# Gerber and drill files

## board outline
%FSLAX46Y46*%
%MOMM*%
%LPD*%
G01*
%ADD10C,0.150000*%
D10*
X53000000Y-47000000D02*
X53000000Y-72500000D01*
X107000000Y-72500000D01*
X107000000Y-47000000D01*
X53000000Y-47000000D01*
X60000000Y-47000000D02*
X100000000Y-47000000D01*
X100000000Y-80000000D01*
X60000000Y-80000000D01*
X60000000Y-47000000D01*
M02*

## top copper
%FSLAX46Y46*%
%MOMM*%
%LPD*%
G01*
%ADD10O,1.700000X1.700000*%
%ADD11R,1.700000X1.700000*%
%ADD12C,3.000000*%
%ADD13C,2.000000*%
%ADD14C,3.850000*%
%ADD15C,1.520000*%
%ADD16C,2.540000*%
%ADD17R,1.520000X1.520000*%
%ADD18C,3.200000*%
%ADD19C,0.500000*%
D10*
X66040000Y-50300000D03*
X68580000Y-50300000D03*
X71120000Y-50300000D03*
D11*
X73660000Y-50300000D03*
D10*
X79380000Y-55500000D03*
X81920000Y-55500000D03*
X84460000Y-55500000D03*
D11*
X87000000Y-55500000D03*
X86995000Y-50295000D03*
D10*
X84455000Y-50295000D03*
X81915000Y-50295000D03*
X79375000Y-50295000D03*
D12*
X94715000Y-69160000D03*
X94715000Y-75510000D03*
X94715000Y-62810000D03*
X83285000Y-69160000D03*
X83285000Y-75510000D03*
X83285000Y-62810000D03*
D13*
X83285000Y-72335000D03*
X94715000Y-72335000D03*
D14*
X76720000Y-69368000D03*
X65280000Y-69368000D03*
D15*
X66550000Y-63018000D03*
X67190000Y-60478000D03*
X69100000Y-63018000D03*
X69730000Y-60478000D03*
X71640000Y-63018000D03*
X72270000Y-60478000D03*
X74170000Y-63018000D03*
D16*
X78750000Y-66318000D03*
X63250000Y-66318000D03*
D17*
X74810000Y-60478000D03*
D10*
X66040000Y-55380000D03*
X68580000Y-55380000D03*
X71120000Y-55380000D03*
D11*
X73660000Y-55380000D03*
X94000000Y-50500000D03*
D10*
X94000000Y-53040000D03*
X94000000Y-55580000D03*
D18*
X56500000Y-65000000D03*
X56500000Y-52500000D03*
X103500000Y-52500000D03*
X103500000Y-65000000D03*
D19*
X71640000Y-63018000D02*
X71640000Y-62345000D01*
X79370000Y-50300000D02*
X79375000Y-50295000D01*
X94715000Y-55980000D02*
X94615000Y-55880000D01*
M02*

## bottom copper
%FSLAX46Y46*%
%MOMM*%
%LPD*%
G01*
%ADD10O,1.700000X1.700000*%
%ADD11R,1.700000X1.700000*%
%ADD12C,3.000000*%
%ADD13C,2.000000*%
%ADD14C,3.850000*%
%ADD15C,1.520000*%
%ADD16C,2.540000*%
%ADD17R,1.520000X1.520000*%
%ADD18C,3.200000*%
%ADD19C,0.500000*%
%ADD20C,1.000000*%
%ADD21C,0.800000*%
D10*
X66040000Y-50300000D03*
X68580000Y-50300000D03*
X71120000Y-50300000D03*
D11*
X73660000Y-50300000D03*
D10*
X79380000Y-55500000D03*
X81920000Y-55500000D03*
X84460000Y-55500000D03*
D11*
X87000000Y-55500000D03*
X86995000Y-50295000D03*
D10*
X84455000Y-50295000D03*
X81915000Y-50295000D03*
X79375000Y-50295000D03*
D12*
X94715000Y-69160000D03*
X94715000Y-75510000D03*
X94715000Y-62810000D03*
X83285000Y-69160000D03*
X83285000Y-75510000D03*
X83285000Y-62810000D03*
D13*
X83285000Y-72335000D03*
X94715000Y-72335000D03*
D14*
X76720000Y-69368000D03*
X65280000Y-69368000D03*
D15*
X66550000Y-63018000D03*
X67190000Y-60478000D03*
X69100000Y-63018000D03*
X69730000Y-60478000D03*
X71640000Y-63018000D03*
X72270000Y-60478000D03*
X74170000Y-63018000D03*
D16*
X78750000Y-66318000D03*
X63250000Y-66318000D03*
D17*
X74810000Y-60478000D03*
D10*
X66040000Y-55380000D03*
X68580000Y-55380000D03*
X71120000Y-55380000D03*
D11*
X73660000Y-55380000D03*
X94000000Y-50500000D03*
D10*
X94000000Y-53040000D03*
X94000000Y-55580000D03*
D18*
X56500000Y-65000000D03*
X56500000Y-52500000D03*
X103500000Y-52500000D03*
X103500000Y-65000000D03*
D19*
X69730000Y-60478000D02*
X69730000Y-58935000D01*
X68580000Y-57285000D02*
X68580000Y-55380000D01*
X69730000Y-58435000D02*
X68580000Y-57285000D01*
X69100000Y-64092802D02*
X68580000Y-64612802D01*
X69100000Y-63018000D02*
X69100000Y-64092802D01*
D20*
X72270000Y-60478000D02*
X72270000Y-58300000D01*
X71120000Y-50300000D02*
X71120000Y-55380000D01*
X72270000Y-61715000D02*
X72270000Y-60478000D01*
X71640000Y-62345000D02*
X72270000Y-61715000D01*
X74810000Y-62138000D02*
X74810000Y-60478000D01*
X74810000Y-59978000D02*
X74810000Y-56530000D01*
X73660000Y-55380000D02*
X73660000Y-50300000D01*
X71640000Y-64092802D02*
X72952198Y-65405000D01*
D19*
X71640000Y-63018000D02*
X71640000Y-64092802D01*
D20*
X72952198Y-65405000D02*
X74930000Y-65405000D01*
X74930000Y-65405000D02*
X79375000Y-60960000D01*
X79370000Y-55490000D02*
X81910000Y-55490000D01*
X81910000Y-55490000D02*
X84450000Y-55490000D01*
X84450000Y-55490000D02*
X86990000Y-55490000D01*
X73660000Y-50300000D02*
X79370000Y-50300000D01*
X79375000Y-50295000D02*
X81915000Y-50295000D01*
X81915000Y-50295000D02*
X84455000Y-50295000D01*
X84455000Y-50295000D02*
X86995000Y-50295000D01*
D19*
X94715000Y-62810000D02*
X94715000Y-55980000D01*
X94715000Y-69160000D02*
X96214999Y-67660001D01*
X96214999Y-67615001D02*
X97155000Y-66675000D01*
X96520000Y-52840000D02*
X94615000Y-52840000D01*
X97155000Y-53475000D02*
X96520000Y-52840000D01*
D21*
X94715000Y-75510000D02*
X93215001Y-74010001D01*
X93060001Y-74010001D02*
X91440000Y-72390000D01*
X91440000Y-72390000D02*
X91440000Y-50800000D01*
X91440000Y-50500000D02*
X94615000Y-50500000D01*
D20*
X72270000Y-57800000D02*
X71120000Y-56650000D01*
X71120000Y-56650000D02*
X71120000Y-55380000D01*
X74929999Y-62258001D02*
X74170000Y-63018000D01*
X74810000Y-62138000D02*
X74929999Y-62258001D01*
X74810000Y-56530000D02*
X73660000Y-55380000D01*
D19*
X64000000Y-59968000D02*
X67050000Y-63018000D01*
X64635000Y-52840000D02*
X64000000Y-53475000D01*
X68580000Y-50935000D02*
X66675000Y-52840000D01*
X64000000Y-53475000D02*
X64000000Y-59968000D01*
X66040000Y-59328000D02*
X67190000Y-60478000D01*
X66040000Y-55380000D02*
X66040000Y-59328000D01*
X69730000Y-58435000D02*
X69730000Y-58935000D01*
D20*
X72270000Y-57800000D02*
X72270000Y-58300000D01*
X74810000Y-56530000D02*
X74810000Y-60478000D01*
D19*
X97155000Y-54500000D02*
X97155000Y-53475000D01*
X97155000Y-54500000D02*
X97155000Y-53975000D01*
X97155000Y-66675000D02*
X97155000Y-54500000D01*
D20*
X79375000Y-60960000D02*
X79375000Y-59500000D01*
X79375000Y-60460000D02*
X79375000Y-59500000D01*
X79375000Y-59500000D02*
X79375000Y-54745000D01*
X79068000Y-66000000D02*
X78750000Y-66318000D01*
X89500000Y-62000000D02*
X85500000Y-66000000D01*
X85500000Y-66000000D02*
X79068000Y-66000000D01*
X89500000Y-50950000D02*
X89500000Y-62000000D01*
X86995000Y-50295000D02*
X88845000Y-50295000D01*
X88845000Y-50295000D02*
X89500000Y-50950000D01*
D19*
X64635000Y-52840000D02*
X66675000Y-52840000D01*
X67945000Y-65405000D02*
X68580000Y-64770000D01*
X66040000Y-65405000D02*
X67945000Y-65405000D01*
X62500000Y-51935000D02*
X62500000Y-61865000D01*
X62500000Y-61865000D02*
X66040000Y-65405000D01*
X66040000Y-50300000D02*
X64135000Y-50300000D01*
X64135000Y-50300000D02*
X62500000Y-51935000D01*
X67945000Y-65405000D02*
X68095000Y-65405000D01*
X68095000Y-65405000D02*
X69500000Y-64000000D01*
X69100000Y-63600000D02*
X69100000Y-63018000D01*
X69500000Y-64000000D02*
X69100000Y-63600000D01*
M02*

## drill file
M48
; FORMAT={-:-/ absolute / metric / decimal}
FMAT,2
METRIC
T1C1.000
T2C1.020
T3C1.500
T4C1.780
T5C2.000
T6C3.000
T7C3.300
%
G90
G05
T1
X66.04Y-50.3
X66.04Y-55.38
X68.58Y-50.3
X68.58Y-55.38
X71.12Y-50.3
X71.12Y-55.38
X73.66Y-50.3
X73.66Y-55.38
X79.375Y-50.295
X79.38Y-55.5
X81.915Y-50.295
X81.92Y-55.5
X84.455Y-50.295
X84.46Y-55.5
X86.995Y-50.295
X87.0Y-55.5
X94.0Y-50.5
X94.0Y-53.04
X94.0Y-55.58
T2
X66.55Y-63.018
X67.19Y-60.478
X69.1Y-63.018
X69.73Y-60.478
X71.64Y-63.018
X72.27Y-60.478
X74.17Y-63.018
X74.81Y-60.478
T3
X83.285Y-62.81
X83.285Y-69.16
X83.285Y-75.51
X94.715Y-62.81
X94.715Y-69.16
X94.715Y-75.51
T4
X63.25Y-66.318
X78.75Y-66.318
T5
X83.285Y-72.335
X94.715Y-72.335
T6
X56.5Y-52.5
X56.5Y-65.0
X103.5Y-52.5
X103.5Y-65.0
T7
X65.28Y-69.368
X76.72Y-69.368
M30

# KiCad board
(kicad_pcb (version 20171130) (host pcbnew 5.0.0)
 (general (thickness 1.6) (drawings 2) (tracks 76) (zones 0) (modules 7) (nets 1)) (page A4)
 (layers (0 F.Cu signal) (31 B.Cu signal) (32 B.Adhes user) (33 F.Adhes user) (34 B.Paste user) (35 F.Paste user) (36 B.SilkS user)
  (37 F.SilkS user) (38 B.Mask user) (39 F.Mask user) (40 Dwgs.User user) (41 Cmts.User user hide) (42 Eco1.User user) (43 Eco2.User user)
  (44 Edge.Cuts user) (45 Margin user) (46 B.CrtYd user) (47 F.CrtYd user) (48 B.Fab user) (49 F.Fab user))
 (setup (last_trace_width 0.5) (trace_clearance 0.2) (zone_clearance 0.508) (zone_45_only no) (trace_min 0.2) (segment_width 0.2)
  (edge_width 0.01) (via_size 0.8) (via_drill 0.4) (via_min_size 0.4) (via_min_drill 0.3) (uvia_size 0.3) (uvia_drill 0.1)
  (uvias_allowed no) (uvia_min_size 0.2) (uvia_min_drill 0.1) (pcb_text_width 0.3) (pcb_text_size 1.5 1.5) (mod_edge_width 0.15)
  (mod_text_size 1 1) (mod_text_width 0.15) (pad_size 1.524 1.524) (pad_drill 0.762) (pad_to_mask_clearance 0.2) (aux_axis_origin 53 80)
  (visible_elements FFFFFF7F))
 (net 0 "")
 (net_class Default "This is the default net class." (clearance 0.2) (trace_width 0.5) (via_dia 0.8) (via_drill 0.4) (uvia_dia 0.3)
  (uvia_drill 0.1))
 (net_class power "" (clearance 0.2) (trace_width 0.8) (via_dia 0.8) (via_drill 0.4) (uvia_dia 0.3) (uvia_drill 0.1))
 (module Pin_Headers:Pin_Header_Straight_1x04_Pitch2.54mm (layer F.Cu) (at 73.66 50.3 270)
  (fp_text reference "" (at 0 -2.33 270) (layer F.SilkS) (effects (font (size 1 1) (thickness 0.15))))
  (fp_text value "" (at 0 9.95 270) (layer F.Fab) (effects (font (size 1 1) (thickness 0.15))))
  (pad 4 thru_hole oval (at 0 7.62 270) (size 1.7 1.7) (drill 1) (layers *.Cu *.Mask))
  (pad 3 thru_hole oval (at 0 5.08 270) (size 1.7 1.7) (drill 1) (layers *.Cu *.Mask))
  (pad 2 thru_hole oval (at 0 2.54 270) (size 1.7 1.7) (drill 1) (layers *.Cu *.Mask))
  (pad 1 thru_hole rect (at 0 0 270) (size 1.7 1.7) (drill 1) (layers *.Cu *.Mask)))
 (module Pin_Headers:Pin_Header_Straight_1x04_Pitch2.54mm (layer F.Cu) (at 87 55.5 270)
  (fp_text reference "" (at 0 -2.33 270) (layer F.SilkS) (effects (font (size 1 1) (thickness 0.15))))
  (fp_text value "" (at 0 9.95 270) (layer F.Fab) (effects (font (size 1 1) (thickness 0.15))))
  (pad 4 thru_hole oval (at 0 7.62 270) (size 1.7 1.7) (drill 1) (layers *.Cu *.Mask))
  (pad 3 thru_hole oval (at 0 5.08 270) (size 1.7 1.7) (drill 1) (layers *.Cu *.Mask))
  (pad 2 thru_hole oval (at 0 2.54 270) (size 1.7 1.7) (drill 1) (layers *.Cu *.Mask))
  (pad 1 thru_hole rect (at 0 0 270) (size 1.7 1.7) (drill 1) (layers *.Cu *.Mask)))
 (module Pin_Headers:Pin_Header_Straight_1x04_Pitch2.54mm (layer F.Cu) (at 86.995 50.295 270)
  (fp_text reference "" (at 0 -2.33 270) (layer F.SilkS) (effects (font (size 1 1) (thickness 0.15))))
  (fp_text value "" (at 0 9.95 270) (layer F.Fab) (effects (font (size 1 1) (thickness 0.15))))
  (pad 1 thru_hole rect (at 0 0 270) (size 1.7 1.7) (drill 1) (layers *.Cu *.Mask))
  (pad 2 thru_hole oval (at 0 2.54 270) (size 1.7 1.7) (drill 1) (layers *.Cu *.Mask))
  (pad 3 thru_hole oval (at 0 5.08 270) (size 1.7 1.7) (drill 1) (layers *.Cu *.Mask))
  (pad 4 thru_hole oval (at 0 7.62 270) (size 1.7 1.7) (drill 1) (layers *.Cu *.Mask)))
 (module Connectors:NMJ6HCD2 (layer F.Cu) (at 89 59)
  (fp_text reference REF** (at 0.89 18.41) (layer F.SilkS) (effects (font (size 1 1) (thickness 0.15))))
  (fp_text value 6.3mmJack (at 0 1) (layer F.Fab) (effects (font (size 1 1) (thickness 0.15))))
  (pad 6 thru_hole circle (at 5.715 10.16) (size 3 3) (drill 1.5) (layers *.Cu *.Mask))
  (pad 5 thru_hole circle (at 5.715 16.51) (size 3 3) (drill 1.5) (layers *.Cu *.Mask))
  (pad 4 thru_hole circle (at 5.715 3.81) (size 3 3) (drill 1.5) (layers *.Cu *.Mask))
  (pad 3 thru_hole circle (at -5.715 10.16) (size 3 3) (drill 1.5) (layers *.Cu *.Mask))
  (pad 2 thru_hole circle (at -5.715 16.51) (size 3 3) (drill 1.5) (layers *.Cu *.Mask))
  (pad 1 thru_hole circle (at -5.715 3.81) (size 3 3) (drill 1.5) (layers *.Cu *.Mask))
  (pad "" thru_hole circle (at -5.715 13.335) (size 2 2) (drill 2) (layers *.Cu *.Mask))
  (pad "" thru_hole circle (at 5.715 13.335) (size 2 2) (drill 2) (layers *.Cu *.Mask)))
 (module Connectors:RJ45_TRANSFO (layer F.Cu) (at 71 59)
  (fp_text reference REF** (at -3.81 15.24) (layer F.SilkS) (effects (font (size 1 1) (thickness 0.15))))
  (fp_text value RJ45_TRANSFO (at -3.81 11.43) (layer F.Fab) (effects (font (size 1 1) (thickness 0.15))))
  (pad Hole thru_hole circle (at 5.72 10.368) (size 3.85 3.85) (drill 3.3) (layers *.Cu *.SilkS *.Mask))
  (pad Hole thru_hole circle (at -5.72 10.368) (size 3.85 3.85) (drill 3.3) (layers *.Cu *.SilkS *.Mask))
  (pad 8 thru_hole circle (at -4.45 4.018) (size 1.52 1.52) (drill 1.02) (layers *.Cu *.Mask))
  (pad 7 thru_hole circle (at -3.81 1.478) (size 1.52 1.52) (drill 1.02) (layers *.Cu *.Mask))
  (pad 6 thru_hole circle (at -1.9 4.018) (size 1.52 1.52) (drill 1.02) (layers *.Cu *.Mask))
  (pad 5 thru_hole circle (at -1.27 1.478) (size 1.52 1.52) (drill 1.02) (layers *.Cu *.Mask))
  (pad 4 thru_hole circle (at 0.64 4.018) (size 1.52 1.52) (drill 1.02) (layers *.Cu *.Mask))
  (pad 3 thru_hole circle (at 1.27 1.478) (size 1.52 1.52) (drill 1.02) (layers *.Cu *.Mask))
  (pad 2 thru_hole circle (at 3.17 4.018) (size 1.52 1.52) (drill 1.02) (layers *.Cu *.Mask))
  (pad 13 thru_hole circle (at 7.75 7.318) (size 2.54 2.54) (drill 1.78) (layers *.Cu *.SilkS *.Mask))
  (pad 13 thru_hole circle (at -7.75 7.318) (size 2.54 2.54) (drill 1.78) (layers *.Cu *.SilkS *.Mask))
  (pad 1 thru_hole rect (at 3.81 1.478) (size 1.52 1.52) (drill 1.02) (layers *.Cu *.Mask)))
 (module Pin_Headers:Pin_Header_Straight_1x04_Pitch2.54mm (layer F.Cu) (at 73.66 55.38 270)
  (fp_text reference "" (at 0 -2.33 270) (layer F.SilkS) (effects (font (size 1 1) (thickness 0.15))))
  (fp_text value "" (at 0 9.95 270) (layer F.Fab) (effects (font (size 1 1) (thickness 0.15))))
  (pad 4 thru_hole oval (at 0 7.62 270) (size 1.7 1.7) (drill 1) (layers *.Cu *.Mask))
  (pad 3 thru_hole oval (at 0 5.08 270) (size 1.7 1.7) (drill 1) (layers *.Cu *.Mask))
  (pad 2 thru_hole oval (at 0 2.54 270) (size 1.7 1.7) (drill 1) (layers *.Cu *.Mask))
  (pad 1 thru_hole rect (at 0 0 270) (size 1.7 1.7) (drill 1) (layers *.Cu *.Mask)))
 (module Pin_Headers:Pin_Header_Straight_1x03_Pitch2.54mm (layer F.Cu) (at 94 50.5)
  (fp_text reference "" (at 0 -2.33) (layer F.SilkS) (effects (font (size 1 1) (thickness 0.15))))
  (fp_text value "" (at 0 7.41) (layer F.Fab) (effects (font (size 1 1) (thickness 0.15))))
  (pad 1 thru_hole rect (at 0 0) (size 1.7 1.7) (drill 1) (layers *.Cu *.Mask))
  (pad 2 thru_hole oval (at 0 2.54) (size 1.7 1.7) (drill 1) (layers *.Cu *.Mask))
  (pad 3 thru_hole oval (at 0 5.08) (size 1.7 1.7) (drill 1) (layers *.Cu *.Mask)))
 (gr_poly (pts (xy 53 47) (xy 53 72.5) (xy 107 72.5) (xy 107 47)) (layer Edge.Cuts) (width 0.15))
 (gr_poly (pts (xy 60 47) (xy 100 47) (xy 100 80) (xy 60 80)) (layer Edge.Cuts) (width 0.15))
 (segment (start 69.73 60.478) (end 69.73 58.935) (width 0.5) (layer B.Cu) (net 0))
 (segment (start 68.58 57.285) (end 68.58 55.38) (width 0.5) (layer B.Cu) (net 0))
 (segment (start 69.73 58.435) (end 68.58 57.285) (width 0.5) (layer B.Cu) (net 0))
 (segment (start 69.1 64.092802) (end 68.58 64.612802) (width 0.5) (layer B.Cu) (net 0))
 (segment (start 69.1 63.018) (end 69.1 64.092802) (width 0.5) (layer B.Cu) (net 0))
 (segment (start 72.27 60.478) (end 72.27 58.3) (width 1) (layer B.Cu) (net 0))
 (segment (start 71.12 50.3) (end 71.12 55.38) (width 1) (layer B.Cu) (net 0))
 (segment (start 71.64 63.018) (end 71.64 62.345) (width 0.5) (layer F.Cu) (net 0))
 (segment (start 72.27 61.715) (end 72.27 60.478) (width 1) (layer B.Cu) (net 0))
 (segment (start 71.64 62.345) (end 72.27 61.715) (width 1) (layer B.Cu) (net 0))
 (segment (start 74.81 62.138) (end 74.81 60.478) (width 1) (layer B.Cu) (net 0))
 (segment (start 74.81 59.978) (end 74.81 56.53) (width 1) (layer B.Cu) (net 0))
 (segment (start 73.66 55.38) (end 73.66 50.3) (width 1) (layer B.Cu) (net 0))
 (segment (start 71.64 64.092802) (end 72.952198 65.405) (width 1) (layer B.Cu) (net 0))
 (segment (start 71.64 63.018) (end 71.64 64.092802) (width 0.5) (layer B.Cu) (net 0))
 (segment (start 72.952198 65.405) (end 74.93 65.405) (width 1) (layer B.Cu) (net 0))
 (segment (start 74.93 65.405) (end 79.375 60.96) (width 1) (layer B.Cu) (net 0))
 (segment (start 79.37 55.49) (end 81.91 55.49) (width 1) (layer B.Cu) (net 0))
 (segment (start 81.91 55.49) (end 84.45 55.49) (width 1) (layer B.Cu) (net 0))
 (segment (start 84.45 55.49) (end 86.99 55.49) (width 1) (layer B.Cu) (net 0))
 (segment (start 79.37 50.3) (end 79.375 50.295) (width 0.5) (layer F.Cu) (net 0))
 (segment (start 73.66 50.3) (end 79.37 50.3) (width 1) (layer B.Cu) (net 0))
 (segment (start 79.375 50.295) (end 81.915 50.295) (width 1) (layer B.Cu) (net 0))
 (segment (start 81.915 50.295) (end 84.455 50.295) (width 1) (layer B.Cu) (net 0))
 (segment (start 84.455 50.295) (end 86.995 50.295) (width 1) (layer B.Cu) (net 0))
 (segment (start 94.715 55.98) (end 94.615 55.88) (width 0.5) (layer F.Cu) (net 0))
 (segment (start 94.715 62.81) (end 94.715 55.98) (width 0.5) (layer B.Cu) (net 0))
 (segment (start 94.715 69.16) (end 96.214999 67.660001) (width 0.5) (layer B.Cu) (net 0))
 (segment (start 96.214999 67.615001) (end 97.155 66.675) (width 0.5) (layer B.Cu) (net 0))
 (segment (start 96.52 52.84) (end 94.615 52.84) (width 0.5) (layer B.Cu) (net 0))
 (segment (start 97.155 53.475) (end 96.52 52.84) (width 0.5) (layer B.Cu) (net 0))
 (segment (start 94.715 75.51) (end 93.215001 74.010001) (width 0.8) (layer B.Cu) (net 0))
 (segment (start 93.060001 74.010001) (end 91.44 72.39) (width 0.8) (layer B.Cu) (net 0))
 (segment (start 91.44 72.39) (end 91.44 50.8) (width 0.8) (layer B.Cu) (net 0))
 (segment (start 91.44 50.5) (end 94.615 50.5) (width 0.8) (layer B.Cu) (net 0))
 (segment (start 72.27 57.8) (end 71.12 56.65) (width 1) (layer B.Cu) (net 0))
 (segment (start 71.12 56.65) (end 71.12 55.38) (width 1) (layer B.Cu) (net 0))
 (segment (start 74.929999 62.258001) (end 74.17 63.018) (width 1) (layer B.Cu) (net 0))
 (segment (start 74.81 62.138) (end 74.929999 62.258001) (width 1) (layer B.Cu) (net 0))
 (segment (start 74.81 56.53) (end 73.66 55.38) (width 1) (layer B.Cu) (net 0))
 (via (at 56.5 65) (size 3.2) (drill 3) (layers F.Cu B.Cu) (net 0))
 (via (at 56.5 52.5) (size 3.2) (drill 3) (layers F.Cu B.Cu) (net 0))
 (via (at 103.5 52.5) (size 3.2) (drill 3) (layers F.Cu B.Cu) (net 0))
 (via (at 103.5 65) (size 3.2) (drill 3) (layers F.Cu B.Cu) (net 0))
 (segment (start 64 59.968) (end 67.05 63.018) (width 0.5) (layer B.Cu) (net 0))
 (segment (start 64.635 52.84) (end 64 53.475) (width 0.5) (layer B.Cu) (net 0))
 (segment (start 68.58 50.935) (end 66.675 52.84) (width 0.5) (layer B.Cu) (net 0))
 (segment (start 64 53.475) (end 64 59.968) (width 0.5) (layer B.Cu) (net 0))
 (segment (start 66.04 59.328) (end 67.19 60.478) (width 0.5) (layer B.Cu) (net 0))
 (segment (start 66.04 55.38) (end 66.04 59.328) (width 0.5) (layer B.Cu) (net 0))
 (segment (start 69.73 58.435) (end 69.73 58.935) (width 0.5) (layer B.Cu) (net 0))
 (segment (start 72.27 57.8) (end 72.27 58.3) (width 1) (layer B.Cu) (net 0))
 (segment (start 74.81 56.53) (end 74.81 60.478) (width 1) (layer B.Cu) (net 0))
 (segment (start 97.155 54.5) (end 97.155 53.475) (width 0.5) (layer B.Cu) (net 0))
 (segment (start 97.155 54.5) (end 97.155 53.975) (width 0.5) (layer B.Cu) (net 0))
 (segment (start 97.155 66.675) (end 97.155 54.5) (width 0.5) (layer B.Cu) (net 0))
 (segment (start 79.375 60.96) (end 79.375 59.5) (width 1) (layer B.Cu) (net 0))
 (segment (start 79.375 60.46) (end 79.375 59.5) (width 1) (layer B.Cu) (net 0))
 (segment (start 79.375 59.5) (end 79.375 54.745) (width 1) (layer B.Cu) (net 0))
 (segment (start 79.068 66) (end 78.75 66.318) (width 1) (layer B.Cu) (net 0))
 (segment (start 89.5 62) (end 85.5 66) (width 1) (layer B.Cu) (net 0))
 (segment (start 85.5 66) (end 79.068 66) (width 1) (layer B.Cu) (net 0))
 (segment (start 89.5 50.95) (end 89.5 62) (width 1) (layer B.Cu) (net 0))
 (segment (start 86.995 50.295) (end 88.845 50.295) (width 1) (layer B.Cu) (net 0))
 (segment (start 88.845 50.295) (end 89.5 50.95) (width 1) (layer B.Cu) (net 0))
 (segment (start 64.635 52.84) (end 66.675 52.84) (width 0.5) (layer B.Cu) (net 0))
 (segment (start 67.945 65.405) (end 68.58 64.77) (width 0.5) (layer B.Cu) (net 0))
 (segment (start 66.04 65.405) (end 67.945 65.405) (width 0.5) (layer B.Cu) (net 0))
 (segment (start 62.5 51.935) (end 62.5 61.865) (width 0.5) (layer B.Cu) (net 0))
 (segment (start 62.5 61.865) (end 66.04 65.405) (width 0.5) (layer B.Cu) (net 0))
 (segment (start 66.04 50.3) (end 64.135 50.3) (width 0.5) (layer B.Cu) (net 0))
 (segment (start 64.135 50.3) (end 62.5 51.935) (width 0.5) (layer B.Cu) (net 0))
 (segment (start 67.945 65.405) (end 68.095 65.405) (width 0.5) (layer B.Cu) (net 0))
 (segment (start 68.095 65.405) (end 69.5 64) (width 0.5) (layer B.Cu) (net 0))
 (segment (start 69.1 63.6) (end 69.1 63.018) (width 0.5) (layer B.Cu) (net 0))
 (segment (start 69.5 64) (end 69.1 63.6) (width 0.5) (layer B.Cu) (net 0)))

